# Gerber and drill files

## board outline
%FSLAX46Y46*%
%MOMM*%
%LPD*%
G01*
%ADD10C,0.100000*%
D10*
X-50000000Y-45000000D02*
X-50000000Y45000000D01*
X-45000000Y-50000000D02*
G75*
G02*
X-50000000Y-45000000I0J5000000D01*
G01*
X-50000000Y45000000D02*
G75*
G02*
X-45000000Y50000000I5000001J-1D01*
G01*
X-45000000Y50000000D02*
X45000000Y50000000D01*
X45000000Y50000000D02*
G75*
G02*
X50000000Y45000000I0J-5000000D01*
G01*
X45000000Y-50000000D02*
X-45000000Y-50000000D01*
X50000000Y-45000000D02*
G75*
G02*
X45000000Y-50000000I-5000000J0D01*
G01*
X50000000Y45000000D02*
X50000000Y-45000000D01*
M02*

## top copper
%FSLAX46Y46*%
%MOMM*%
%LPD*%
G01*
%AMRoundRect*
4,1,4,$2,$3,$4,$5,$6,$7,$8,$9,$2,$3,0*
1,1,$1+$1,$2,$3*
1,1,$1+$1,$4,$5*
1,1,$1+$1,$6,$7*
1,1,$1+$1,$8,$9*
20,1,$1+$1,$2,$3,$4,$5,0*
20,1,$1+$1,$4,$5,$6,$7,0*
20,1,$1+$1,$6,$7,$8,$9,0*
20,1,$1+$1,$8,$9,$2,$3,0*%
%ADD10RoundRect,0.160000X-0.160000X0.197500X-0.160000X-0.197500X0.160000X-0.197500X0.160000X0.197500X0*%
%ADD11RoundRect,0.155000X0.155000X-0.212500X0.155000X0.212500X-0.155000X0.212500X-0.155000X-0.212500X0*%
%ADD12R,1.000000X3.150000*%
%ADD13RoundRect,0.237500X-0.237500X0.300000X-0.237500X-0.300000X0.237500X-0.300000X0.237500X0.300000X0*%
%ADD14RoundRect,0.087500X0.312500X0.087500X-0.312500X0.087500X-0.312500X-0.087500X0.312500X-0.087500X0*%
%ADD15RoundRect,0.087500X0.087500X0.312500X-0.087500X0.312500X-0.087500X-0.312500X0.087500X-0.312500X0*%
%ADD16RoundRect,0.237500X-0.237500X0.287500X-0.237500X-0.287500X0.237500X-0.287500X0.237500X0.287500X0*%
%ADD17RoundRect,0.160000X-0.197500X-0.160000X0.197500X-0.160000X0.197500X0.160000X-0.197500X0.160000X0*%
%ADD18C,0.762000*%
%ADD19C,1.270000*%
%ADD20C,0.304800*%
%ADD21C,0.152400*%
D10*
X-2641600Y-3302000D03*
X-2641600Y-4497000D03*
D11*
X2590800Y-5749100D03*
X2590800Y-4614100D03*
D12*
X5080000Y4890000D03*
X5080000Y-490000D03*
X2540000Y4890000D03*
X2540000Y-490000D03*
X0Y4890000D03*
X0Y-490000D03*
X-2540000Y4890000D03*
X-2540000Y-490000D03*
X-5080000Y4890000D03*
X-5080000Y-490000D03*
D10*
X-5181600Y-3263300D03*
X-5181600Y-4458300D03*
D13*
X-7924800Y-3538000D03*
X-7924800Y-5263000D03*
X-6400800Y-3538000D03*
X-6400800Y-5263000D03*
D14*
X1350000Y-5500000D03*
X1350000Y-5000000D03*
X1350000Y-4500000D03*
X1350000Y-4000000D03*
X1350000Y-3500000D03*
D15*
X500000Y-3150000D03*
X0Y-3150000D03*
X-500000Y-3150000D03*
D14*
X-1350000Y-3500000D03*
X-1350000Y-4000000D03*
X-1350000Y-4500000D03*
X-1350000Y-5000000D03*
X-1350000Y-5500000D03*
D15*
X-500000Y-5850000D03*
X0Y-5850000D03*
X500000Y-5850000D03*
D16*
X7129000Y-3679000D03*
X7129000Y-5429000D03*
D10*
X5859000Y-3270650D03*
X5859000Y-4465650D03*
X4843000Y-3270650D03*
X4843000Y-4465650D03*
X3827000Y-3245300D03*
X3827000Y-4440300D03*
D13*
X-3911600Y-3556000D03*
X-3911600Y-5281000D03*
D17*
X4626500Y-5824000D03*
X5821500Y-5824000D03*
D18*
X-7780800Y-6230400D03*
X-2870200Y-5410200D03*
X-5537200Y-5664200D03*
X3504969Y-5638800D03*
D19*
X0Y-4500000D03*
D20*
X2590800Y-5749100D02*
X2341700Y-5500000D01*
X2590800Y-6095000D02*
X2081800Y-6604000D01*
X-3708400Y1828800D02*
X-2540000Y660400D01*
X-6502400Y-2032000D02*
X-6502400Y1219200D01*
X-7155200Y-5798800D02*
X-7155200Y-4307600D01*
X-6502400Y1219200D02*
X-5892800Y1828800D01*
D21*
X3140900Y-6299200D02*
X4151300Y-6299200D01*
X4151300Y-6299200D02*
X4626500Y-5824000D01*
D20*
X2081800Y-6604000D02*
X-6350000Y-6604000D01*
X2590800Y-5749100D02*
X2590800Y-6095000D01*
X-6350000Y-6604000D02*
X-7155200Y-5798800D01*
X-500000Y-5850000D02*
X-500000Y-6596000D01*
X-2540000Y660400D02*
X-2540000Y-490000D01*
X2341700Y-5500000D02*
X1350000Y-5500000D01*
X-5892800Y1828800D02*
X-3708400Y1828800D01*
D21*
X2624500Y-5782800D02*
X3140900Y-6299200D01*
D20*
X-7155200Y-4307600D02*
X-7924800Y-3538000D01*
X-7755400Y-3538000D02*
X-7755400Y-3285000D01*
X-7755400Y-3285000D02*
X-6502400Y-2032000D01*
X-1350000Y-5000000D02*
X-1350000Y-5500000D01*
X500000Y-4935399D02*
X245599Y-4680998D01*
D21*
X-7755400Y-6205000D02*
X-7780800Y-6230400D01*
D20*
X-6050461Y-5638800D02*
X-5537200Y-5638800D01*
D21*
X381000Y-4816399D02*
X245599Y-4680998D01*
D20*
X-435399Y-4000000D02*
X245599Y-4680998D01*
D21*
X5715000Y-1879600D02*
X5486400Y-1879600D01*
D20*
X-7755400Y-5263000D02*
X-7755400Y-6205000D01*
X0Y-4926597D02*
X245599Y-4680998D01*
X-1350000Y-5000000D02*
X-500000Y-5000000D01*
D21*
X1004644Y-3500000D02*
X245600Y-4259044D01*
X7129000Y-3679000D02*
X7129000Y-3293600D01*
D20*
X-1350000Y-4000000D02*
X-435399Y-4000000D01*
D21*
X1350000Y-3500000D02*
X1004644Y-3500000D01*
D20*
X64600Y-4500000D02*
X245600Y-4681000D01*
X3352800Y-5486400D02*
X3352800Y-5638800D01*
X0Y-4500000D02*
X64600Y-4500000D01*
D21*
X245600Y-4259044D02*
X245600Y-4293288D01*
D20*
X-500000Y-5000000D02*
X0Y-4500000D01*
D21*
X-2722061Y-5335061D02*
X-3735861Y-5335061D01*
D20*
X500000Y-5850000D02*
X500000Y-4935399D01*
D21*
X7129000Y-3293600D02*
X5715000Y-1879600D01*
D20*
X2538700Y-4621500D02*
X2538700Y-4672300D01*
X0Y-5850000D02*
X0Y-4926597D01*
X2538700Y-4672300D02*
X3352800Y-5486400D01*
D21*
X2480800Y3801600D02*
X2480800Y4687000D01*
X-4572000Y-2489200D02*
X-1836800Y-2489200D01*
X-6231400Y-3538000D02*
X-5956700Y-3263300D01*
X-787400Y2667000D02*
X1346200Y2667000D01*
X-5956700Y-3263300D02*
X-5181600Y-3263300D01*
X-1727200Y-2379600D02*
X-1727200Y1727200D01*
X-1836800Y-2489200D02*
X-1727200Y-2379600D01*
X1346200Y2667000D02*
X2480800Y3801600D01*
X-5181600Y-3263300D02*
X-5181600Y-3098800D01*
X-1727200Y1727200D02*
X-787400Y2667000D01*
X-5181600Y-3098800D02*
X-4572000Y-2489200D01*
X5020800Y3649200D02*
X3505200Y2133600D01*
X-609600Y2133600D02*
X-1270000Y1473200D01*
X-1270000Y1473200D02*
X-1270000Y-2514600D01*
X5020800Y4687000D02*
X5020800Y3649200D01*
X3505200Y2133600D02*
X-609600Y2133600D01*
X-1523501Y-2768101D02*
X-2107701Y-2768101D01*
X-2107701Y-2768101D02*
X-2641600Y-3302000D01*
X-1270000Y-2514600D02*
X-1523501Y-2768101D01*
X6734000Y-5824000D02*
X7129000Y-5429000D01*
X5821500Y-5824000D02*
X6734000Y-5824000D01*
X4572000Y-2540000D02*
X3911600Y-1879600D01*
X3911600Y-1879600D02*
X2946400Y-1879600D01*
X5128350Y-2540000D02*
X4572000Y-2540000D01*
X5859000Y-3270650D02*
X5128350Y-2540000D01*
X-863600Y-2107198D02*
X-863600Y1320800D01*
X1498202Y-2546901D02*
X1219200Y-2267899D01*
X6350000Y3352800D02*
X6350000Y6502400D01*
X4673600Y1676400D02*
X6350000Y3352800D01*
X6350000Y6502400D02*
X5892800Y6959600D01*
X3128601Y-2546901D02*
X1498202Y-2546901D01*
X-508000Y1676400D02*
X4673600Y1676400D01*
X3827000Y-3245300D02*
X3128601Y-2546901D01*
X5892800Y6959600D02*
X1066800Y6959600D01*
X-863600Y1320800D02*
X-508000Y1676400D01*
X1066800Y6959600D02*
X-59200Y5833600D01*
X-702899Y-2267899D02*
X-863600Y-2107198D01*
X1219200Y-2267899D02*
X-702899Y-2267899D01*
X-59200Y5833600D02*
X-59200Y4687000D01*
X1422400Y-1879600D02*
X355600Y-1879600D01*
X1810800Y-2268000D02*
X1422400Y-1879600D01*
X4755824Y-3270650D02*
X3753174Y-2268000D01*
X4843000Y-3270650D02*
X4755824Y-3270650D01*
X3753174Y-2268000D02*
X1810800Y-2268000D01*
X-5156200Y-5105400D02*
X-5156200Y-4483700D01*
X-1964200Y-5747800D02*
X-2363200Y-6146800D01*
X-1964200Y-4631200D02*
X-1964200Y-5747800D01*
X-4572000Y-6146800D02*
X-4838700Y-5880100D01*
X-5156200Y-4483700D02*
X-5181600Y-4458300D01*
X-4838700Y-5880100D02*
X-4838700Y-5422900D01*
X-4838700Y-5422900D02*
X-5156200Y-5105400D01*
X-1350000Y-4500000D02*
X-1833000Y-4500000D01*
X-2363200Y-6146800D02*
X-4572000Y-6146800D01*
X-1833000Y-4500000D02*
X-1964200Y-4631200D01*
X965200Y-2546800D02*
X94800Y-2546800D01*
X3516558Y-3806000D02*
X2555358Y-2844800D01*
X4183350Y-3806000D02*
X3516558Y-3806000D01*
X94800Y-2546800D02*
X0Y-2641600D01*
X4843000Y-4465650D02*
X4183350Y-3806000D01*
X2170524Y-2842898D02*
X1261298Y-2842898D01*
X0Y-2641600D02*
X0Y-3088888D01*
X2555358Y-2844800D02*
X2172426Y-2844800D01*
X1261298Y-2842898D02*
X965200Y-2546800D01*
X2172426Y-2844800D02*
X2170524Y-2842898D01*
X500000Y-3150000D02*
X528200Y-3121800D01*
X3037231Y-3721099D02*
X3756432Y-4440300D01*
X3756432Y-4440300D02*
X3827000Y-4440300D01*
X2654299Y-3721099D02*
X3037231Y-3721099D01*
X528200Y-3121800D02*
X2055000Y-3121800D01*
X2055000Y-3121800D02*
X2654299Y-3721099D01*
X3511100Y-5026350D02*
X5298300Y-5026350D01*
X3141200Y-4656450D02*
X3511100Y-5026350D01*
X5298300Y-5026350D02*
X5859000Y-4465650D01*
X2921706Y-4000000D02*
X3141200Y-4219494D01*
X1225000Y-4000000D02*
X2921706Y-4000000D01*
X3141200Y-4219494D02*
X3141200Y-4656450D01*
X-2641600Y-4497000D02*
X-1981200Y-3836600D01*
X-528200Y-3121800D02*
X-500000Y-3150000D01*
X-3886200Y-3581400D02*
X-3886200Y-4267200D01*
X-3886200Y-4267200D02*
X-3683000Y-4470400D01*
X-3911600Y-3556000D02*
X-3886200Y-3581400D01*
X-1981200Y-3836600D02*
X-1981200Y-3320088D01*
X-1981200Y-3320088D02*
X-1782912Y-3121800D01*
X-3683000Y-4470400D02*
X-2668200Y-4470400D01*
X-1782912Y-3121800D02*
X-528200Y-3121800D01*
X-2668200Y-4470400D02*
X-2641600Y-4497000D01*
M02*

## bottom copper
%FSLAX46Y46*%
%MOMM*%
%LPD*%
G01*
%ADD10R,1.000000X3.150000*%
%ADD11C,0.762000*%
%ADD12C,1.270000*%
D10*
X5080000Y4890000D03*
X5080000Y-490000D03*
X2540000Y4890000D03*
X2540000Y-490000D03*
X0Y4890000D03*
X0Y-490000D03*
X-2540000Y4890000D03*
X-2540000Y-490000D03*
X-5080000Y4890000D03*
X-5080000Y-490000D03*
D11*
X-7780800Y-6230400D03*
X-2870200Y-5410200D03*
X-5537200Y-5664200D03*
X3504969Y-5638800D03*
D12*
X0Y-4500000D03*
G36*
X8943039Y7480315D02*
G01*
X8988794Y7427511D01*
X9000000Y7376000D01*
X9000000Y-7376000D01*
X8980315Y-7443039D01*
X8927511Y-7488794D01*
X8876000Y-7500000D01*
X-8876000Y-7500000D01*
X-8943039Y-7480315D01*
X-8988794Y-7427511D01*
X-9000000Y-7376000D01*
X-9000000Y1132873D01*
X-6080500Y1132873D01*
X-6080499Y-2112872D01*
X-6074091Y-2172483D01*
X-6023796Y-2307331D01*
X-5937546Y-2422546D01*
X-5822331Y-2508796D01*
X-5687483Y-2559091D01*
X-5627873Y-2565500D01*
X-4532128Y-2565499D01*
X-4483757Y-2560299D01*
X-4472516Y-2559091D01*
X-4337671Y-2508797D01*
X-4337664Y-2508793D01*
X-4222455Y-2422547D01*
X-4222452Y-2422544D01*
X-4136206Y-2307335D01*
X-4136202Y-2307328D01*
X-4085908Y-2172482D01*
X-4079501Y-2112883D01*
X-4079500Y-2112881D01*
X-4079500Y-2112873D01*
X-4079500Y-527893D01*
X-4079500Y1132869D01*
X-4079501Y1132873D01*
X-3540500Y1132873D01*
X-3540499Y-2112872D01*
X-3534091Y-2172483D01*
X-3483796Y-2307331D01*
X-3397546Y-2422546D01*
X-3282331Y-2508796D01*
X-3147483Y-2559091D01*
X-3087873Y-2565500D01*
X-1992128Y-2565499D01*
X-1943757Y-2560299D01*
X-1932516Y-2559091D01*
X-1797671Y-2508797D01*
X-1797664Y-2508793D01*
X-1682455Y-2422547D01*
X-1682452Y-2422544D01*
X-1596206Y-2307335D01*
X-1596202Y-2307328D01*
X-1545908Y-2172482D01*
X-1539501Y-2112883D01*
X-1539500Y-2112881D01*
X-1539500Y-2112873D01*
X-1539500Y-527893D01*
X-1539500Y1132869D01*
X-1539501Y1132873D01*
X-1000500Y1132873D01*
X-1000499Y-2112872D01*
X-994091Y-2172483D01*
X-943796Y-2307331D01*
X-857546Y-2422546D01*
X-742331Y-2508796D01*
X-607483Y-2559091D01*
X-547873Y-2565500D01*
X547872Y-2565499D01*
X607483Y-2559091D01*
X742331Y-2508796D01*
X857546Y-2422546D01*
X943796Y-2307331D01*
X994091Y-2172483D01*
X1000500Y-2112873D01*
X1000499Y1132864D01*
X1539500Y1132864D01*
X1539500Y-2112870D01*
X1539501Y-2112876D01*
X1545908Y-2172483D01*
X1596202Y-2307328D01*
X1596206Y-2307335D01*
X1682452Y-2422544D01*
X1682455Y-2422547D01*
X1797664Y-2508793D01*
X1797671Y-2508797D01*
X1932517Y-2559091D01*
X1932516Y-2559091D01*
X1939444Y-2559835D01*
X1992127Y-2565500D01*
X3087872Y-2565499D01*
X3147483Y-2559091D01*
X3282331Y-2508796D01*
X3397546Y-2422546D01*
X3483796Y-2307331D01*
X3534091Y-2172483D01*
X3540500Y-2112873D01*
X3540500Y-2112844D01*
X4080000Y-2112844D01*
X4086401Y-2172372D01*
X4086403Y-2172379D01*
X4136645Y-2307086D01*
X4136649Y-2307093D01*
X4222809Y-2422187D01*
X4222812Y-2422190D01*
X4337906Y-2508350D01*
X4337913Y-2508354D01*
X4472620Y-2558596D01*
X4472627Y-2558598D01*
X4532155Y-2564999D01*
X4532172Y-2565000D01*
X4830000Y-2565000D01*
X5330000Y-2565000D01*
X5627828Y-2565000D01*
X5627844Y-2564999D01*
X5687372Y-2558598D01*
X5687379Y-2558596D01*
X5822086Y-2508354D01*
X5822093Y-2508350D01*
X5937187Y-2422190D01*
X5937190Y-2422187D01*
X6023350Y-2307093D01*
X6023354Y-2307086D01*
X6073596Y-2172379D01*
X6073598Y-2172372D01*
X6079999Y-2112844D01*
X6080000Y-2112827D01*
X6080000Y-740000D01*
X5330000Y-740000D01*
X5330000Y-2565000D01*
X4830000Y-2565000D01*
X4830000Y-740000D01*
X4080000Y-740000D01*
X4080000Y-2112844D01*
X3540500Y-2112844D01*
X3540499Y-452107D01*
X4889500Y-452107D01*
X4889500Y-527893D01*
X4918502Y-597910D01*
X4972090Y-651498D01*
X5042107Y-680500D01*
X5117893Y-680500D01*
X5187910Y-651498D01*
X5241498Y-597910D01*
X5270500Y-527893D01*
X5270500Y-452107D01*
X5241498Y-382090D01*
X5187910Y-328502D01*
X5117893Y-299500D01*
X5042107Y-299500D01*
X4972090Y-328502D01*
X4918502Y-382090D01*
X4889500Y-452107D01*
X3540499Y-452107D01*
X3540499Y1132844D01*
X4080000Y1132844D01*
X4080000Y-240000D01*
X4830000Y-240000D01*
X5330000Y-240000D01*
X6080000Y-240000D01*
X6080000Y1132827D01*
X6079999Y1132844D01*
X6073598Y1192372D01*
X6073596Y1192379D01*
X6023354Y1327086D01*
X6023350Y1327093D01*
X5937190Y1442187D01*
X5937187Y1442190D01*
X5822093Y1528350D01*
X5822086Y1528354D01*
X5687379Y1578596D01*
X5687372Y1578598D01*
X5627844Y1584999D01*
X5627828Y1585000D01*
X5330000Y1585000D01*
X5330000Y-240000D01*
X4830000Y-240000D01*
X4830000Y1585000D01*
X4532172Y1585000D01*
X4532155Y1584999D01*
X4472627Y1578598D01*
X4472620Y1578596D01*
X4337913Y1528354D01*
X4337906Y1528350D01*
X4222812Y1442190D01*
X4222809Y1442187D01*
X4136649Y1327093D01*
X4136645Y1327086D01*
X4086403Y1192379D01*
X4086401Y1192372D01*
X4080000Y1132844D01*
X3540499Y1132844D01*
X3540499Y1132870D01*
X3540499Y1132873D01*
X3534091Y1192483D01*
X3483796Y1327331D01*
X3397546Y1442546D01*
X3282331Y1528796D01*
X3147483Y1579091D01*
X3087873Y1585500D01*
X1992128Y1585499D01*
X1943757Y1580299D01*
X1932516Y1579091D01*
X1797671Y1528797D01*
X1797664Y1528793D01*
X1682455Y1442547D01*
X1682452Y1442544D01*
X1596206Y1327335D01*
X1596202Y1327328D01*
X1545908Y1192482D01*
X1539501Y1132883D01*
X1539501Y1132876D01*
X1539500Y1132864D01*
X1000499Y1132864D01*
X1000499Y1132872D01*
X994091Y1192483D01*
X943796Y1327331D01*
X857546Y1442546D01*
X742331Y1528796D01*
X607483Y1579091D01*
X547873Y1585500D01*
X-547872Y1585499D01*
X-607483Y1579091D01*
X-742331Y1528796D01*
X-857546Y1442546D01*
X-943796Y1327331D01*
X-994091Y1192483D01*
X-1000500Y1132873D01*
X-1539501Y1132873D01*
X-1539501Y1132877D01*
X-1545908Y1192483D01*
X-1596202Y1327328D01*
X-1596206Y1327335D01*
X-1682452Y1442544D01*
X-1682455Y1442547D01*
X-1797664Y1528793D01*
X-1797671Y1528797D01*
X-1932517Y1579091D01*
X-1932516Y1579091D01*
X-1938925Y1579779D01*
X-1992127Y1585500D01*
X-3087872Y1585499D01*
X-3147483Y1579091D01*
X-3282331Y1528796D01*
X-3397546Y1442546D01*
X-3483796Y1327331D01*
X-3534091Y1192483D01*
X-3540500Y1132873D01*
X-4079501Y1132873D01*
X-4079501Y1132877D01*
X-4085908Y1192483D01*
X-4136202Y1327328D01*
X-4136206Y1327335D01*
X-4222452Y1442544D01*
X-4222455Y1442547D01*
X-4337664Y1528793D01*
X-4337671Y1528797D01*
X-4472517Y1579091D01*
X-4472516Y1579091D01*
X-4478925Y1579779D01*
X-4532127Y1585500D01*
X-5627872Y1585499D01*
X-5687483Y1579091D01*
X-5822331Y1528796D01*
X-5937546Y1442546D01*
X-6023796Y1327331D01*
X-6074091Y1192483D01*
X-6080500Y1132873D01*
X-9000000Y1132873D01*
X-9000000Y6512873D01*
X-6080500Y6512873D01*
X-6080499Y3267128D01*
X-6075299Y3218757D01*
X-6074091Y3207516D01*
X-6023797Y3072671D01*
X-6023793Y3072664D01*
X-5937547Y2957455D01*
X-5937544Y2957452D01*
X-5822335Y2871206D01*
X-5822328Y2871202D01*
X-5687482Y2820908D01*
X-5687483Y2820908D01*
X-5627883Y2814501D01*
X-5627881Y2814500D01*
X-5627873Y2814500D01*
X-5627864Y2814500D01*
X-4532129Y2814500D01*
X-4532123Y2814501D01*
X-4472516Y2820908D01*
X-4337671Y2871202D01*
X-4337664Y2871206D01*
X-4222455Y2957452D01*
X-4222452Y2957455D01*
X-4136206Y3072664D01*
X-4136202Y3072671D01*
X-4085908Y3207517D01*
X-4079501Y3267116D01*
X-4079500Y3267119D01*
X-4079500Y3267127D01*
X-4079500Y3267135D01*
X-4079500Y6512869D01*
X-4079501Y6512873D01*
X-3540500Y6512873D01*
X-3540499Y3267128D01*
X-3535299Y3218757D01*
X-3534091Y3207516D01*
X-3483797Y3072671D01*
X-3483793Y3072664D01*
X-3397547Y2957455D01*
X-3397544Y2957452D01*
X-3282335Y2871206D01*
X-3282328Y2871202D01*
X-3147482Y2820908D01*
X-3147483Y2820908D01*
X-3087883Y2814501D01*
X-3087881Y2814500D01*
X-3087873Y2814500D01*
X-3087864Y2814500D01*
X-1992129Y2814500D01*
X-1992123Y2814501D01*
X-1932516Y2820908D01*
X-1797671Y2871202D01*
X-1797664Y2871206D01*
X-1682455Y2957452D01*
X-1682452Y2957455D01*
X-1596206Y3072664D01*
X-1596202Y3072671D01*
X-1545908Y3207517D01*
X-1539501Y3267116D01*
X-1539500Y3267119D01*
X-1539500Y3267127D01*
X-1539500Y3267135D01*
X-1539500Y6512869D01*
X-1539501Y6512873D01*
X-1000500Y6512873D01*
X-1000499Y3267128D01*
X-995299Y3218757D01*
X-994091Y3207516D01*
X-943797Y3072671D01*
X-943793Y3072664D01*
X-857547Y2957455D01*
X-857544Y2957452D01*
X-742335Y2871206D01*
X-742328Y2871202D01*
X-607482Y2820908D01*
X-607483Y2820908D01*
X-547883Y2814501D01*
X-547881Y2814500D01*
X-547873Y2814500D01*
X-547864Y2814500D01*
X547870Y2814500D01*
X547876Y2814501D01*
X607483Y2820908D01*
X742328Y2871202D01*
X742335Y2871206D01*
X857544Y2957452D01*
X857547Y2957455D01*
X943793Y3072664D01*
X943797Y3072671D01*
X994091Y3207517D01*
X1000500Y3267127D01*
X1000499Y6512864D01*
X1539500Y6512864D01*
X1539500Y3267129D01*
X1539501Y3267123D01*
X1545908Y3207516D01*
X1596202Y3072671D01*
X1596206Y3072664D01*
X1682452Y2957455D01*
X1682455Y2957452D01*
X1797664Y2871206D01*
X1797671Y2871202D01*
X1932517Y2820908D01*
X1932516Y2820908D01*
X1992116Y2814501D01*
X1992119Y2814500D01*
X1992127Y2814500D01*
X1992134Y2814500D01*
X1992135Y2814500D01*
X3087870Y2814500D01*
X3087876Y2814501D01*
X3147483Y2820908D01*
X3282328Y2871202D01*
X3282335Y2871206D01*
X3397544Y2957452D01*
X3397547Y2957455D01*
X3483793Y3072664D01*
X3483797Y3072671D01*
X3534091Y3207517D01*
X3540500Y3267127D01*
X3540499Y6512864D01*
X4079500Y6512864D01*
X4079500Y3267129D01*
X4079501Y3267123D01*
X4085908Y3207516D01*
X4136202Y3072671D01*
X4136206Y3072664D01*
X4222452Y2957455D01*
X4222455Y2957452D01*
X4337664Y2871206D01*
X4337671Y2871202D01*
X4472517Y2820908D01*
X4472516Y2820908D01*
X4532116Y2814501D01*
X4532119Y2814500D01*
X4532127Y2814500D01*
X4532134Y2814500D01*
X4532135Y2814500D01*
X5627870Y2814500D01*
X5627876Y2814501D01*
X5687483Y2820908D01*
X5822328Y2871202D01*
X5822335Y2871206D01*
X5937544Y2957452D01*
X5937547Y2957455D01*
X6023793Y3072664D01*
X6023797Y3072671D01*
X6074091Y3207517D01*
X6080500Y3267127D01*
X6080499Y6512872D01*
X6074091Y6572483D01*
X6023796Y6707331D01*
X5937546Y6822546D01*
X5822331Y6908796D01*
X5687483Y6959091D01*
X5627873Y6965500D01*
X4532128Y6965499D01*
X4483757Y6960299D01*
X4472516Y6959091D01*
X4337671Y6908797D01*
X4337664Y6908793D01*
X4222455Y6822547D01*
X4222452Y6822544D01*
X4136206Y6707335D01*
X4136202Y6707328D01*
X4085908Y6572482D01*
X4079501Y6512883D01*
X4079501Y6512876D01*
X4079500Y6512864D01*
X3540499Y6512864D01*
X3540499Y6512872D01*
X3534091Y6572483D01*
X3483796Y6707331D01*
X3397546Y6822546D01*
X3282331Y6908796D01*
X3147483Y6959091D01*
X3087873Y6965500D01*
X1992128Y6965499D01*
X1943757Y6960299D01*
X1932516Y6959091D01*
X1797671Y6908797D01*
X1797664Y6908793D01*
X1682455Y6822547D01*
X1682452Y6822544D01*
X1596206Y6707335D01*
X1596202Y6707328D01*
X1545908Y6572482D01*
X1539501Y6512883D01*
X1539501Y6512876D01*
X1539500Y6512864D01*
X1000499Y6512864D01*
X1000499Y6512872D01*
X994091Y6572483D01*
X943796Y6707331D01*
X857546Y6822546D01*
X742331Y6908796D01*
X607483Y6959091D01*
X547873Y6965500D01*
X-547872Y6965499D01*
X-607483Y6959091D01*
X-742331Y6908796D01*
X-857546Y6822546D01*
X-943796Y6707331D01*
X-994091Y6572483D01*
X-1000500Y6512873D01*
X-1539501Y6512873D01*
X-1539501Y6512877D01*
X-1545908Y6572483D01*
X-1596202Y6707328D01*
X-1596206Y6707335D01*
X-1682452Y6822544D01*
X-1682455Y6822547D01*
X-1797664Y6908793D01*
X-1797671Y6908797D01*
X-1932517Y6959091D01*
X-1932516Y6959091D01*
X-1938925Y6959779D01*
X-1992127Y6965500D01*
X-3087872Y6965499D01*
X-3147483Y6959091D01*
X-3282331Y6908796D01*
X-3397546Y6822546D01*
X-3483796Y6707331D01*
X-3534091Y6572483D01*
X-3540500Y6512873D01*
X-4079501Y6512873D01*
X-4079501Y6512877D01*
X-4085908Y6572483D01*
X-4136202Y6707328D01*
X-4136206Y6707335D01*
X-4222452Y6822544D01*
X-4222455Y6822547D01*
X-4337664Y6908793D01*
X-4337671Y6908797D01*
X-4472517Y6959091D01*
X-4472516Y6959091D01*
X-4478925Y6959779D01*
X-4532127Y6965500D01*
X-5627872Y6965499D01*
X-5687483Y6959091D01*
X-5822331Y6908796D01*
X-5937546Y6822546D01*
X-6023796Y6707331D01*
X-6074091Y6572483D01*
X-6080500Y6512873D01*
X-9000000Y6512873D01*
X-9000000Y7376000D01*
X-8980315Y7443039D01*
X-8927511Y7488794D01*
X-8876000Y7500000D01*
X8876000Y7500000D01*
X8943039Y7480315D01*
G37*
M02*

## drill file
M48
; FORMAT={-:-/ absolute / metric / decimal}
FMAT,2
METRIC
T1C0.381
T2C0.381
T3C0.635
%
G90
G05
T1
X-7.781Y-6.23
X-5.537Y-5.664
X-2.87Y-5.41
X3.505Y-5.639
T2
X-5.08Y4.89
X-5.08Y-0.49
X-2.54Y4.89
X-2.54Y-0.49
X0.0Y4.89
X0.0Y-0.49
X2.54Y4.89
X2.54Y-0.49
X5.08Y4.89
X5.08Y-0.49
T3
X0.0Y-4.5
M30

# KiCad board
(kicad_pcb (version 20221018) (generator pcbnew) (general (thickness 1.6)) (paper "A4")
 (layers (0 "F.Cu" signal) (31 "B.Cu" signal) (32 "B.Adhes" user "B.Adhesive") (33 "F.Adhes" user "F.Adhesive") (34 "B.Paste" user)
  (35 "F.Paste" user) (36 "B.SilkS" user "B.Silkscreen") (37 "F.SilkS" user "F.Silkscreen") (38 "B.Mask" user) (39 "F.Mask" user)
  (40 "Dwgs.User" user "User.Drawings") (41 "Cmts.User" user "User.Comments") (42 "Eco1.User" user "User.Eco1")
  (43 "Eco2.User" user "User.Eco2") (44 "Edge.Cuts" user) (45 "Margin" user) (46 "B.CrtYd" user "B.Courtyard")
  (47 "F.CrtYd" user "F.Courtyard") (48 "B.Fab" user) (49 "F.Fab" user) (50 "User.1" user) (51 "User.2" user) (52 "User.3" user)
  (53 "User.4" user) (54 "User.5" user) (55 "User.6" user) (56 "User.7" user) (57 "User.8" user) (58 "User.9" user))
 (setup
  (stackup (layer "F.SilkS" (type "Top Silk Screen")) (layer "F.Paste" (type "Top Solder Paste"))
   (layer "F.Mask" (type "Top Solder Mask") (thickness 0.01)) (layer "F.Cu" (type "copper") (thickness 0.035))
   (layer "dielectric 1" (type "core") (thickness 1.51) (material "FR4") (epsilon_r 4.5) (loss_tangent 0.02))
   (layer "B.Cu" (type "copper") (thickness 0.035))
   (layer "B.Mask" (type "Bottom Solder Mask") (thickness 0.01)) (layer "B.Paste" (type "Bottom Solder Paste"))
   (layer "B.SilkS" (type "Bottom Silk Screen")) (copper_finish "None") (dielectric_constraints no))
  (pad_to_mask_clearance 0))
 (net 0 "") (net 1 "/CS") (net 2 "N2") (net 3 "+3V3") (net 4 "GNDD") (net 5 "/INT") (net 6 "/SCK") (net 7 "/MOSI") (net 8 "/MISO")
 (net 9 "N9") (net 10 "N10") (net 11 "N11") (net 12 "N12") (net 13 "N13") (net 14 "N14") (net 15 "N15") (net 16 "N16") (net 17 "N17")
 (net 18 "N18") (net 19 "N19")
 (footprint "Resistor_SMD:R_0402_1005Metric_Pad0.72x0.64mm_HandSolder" (layer "F.Cu") (at -2.6416 3.8995 -90)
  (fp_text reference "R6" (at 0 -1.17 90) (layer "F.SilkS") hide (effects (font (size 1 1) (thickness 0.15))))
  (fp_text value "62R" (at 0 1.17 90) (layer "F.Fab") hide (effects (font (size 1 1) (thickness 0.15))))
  (pad "1" smd roundrect (at -0.5975 0 270) (size 0.715 0.64) (layers "F.Cu" "F.Paste" "F.Mask") (roundrect_rratio 0.25) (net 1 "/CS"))
  (pad "2" smd roundrect (at 0.5975 0 270) (size 0.715 0.64) (layers "F.Cu" "F.Paste" "F.Mask") (roundrect_rratio 0.25) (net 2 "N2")))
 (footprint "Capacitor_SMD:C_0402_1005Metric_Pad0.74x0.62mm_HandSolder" (layer "F.Cu") (at 2.5908 5.1816 90)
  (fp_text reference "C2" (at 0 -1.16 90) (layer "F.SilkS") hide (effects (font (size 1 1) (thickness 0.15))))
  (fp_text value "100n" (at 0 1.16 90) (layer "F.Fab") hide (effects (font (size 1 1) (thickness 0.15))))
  (pad "1" smd roundrect (at -0.5675 0 90) (size 0.735 0.62) (layers "F.Cu" "F.Paste" "F.Mask") (roundrect_rratio 0.25) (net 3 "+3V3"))
  (pad "2" smd roundrect (at 0.5675 0 90) (size 0.735 0.62) (layers "F.Cu" "F.Paste" "F.Mask") (roundrect_rratio 0.25) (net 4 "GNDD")))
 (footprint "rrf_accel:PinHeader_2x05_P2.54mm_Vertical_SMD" (layer "F.Cu") (at 0 -2.2 -90)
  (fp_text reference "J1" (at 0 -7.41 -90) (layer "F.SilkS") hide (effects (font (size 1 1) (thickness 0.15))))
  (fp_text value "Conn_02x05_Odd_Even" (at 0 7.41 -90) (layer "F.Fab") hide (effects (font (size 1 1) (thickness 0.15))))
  (pad "1" thru_hole rect (at -2.69 -5.08 270) (size 3.15 1) (drill 0.381) (layers "*.Cu" "F.Paste" "F.Mask") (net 1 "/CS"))
  (pad "2" thru_hole rect (at 2.69 -5.08 270) (size 3.15 1) (drill 0.381) (layers "*.Cu" "F.Paste" "F.Mask") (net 4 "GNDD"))
  (pad "3" thru_hole rect (at -2.69 -2.54 270) (size 3.15 1) (drill 0.381) (layers "*.Cu" "F.Paste" "F.Mask") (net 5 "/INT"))
  (pad "4" thru_hole rect (at 2.69 -2.54 270) (size 3.15 1) (drill 0.381) (layers "*.Cu" "F.Paste" "F.Mask") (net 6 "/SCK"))
  (pad "5" thru_hole rect (at -2.69 0 270) (size 3.15 1) (drill 0.381) (layers "*.Cu" "F.Paste" "F.Mask") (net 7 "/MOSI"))
  (pad "6" thru_hole rect (at 2.69 0 270) (size 3.15 1) (drill 0.381) (layers "*.Cu" "F.Paste" "F.Mask") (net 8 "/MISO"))
  (pad "7" thru_hole rect (at -2.69 2.54 270) (size 3.15 1) (drill 0.381) (layers "*.Cu" "F.Paste" "F.Mask") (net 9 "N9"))
  (pad "8" thru_hole rect (at 2.69 2.54 270) (size 3.15 1) (drill 0.381) (layers "*.Cu" "F.Paste" "F.Mask") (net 3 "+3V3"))
  (pad "9" thru_hole rect (at -2.69 5.08 270) (size 3.15 1) (drill 0.381) (layers "*.Cu" "F.Paste" "F.Mask") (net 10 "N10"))
  (pad "10" thru_hole rect (at 2.69 5.08 270) (size 3.15 1) (drill 0.381) (layers "*.Cu" "F.Paste" "F.Mask") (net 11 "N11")))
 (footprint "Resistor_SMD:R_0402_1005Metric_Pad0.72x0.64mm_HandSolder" (layer "F.Cu") (at -5.1816 3.8608 -90)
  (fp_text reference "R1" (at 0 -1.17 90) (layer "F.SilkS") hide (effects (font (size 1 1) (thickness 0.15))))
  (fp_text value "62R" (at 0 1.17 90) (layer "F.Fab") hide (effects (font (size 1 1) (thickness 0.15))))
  (pad "1" smd roundrect (at -0.5975 0 270) (size 0.715 0.64) (layers "F.Cu" "F.Paste" "F.Mask") (roundrect_rratio 0.25) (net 5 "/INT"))
  (pad "2" smd roundrect (at 0.5975 0 270) (size 0.715 0.64) (layers "F.Cu" "F.Paste" "F.Mask") (roundrect_rratio 0.25) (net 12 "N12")))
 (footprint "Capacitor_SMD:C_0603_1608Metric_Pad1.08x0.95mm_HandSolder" (layer "F.Cu") (at -7.9248 4.4005 -90)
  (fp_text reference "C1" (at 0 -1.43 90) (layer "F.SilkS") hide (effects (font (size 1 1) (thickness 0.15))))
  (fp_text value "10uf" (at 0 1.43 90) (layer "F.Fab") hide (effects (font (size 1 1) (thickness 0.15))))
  (pad "1" smd roundrect (at -0.8625 0 270) (size 1.075 0.95) (layers "F.Cu" "F.Paste" "F.Mask") (roundrect_rratio 0.25) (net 3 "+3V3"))
  (pad "2" smd roundrect (at 0.8625 0 270) (size 1.075 0.95) (layers "F.Cu" "F.Paste" "F.Mask") (roundrect_rratio 0.25) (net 4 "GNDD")))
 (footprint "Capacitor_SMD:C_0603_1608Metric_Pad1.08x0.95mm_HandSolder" (layer "F.Cu") (at -6.4008 4.4005 -90)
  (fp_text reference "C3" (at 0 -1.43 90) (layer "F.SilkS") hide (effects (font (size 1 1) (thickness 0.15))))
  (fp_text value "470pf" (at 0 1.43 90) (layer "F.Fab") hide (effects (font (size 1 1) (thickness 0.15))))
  (pad "1" smd roundrect (at -0.8625 0 270) (size 1.075 0.95) (layers "F.Cu" "F.Paste" "F.Mask") (roundrect_rratio 0.25) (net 5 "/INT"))
  (pad "2" smd roundrect (at 0.8625 0 270) (size 1.075 0.95) (layers "F.Cu" "F.Paste" "F.Mask") (roundrect_rratio 0.25) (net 4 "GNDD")))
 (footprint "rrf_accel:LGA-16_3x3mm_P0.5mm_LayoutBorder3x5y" (layer "F.Cu") (at 0 4.5 180)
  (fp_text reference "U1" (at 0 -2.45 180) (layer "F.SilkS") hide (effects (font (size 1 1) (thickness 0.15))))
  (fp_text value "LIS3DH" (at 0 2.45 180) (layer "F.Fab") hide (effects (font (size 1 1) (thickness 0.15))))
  (pad "1" smd roundrect (at -1.35 -1 180) (size 0.8 0.35) (layers "F.Cu" "F.Paste" "F.Mask") (roundrect_rratio 0.25) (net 3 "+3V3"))
  (pad "2" smd roundrect (at -1.35 -0.5 180) (size 0.8 0.35) (layers "F.Cu" "F.Paste" "F.Mask") (roundrect_rratio 0.25) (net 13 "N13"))
  (pad "3" smd roundrect (at -1.35 0 180) (size 0.8 0.35) (layers "F.Cu" "F.Paste" "F.Mask") (roundrect_rratio 0.25) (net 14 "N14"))
  (pad "4" smd roundrect (at -1.35 0.5 180) (size 0.8 0.35) (layers "F.Cu" "F.Paste" "F.Mask") (roundrect_rratio 0.25) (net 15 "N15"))
  (pad "5" smd roundrect (at -1.35 1 180) (size 0.8 0.35) (layers "F.Cu" "F.Paste" "F.Mask") (roundrect_rratio 0.25) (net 4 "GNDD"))
  (pad "6" smd roundrect (at -0.5 1.35 180) (size 0.35 0.8) (layers "F.Cu" "F.Paste" "F.Mask") (roundrect_rratio 0.25) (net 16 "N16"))
  (pad "7" smd roundrect (at 0 1.35 180) (size 0.35 0.8) (layers "F.Cu" "F.Paste" "F.Mask") (roundrect_rratio 0.25) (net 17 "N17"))
  (pad "8" smd roundrect (at 0.5 1.35 180) (size 0.35 0.8) (layers "F.Cu" "F.Paste" "F.Mask") (roundrect_rratio 0.25) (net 2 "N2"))
  (pad "9" smd roundrect (at 1.35 1 180) (size 0.8 0.35) (layers "F.Cu" "F.Paste" "F.Mask") (roundrect_rratio 0.25) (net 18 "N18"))
  (pad "10" smd roundrect (at 1.35 0.5 180) (size 0.8 0.35) (layers "F.Cu" "F.Paste" "F.Mask") (roundrect_rratio 0.25) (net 4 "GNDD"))
  (pad "11" smd roundrect (at 1.35 0 180) (size 0.8 0.35) (layers "F.Cu" "F.Paste" "F.Mask") (roundrect_rratio 0.25) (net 12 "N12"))
  (pad "12" smd roundrect (at 1.35 -0.5 180) (size 0.8 0.35) (layers "F.Cu" "F.Paste" "F.Mask") (roundrect_rratio 0.25) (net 4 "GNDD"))
  (pad "13" smd roundrect (at 1.35 -1 180) (size 0.8 0.35) (layers "F.Cu" "F.Paste" "F.Mask") (roundrect_rratio 0.25) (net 4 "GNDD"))
  (pad "14" smd roundrect (at 0.5 -1.35 180) (size 0.35 0.8) (layers "F.Cu" "F.Paste" "F.Mask") (roundrect_rratio 0.25) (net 3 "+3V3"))
  (pad "15" smd roundrect (at 0 -1.35 180) (size 0.35 0.8) (layers "F.Cu" "F.Paste" "F.Mask") (roundrect_rratio 0.25) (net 4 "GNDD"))
  (pad "16" smd roundrect (at -0.5 -1.35 180) (size 0.35 0.8) (layers "F.Cu" "F.Paste" "F.Mask") (roundrect_rratio 0.25) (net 4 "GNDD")))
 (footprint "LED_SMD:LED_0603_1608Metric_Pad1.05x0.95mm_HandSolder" (layer "F.Cu") (at 7.129 4.554 -90)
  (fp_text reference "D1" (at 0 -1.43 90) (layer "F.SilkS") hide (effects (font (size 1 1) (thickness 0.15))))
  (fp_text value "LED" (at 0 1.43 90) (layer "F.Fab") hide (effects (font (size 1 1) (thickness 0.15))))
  (pad "1" smd roundrect (at -0.875 0 270) (size 1.05 0.95) (layers "F.Cu" "F.Paste" "F.Mask") (roundrect_rratio 0.25) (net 4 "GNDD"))
  (pad "2" smd roundrect (at 0.875 0 270) (size 1.05 0.95) (layers "F.Cu" "F.Paste" "F.Mask") (roundrect_rratio 0.25) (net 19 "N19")))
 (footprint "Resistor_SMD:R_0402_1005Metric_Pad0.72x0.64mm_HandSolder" (layer "F.Cu") (at 5.859 3.86815 -90)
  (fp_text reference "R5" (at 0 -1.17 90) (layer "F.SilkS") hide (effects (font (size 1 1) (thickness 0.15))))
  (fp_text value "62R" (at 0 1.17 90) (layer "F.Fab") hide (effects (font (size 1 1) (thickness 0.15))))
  (pad "1" smd roundrect (at -0.5975 0 270) (size 0.715 0.64) (layers "F.Cu" "F.Paste" "F.Mask") (roundrect_rratio 0.25) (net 6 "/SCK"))
  (pad "2" smd roundrect (at 0.5975 0 270) (size 0.715 0.64) (layers "F.Cu" "F.Paste" "F.Mask") (roundrect_rratio 0.25) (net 15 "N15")))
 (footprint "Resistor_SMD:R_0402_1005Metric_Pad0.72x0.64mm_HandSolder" (layer "F.Cu") (at 4.843 3.86815 -90)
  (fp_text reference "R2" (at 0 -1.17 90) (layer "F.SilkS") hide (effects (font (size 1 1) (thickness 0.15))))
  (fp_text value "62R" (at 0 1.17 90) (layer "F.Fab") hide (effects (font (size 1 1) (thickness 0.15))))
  (pad "1" smd roundrect (at -0.5975 0 270) (size 0.715 0.64) (layers "F.Cu" "F.Paste" "F.Mask") (roundrect_rratio 0.25) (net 8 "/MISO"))
  (pad "2" smd roundrect (at 0.5975 0 270) (size 0.715 0.64) (layers "F.Cu" "F.Paste" "F.Mask") (roundrect_rratio 0.25) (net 17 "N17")))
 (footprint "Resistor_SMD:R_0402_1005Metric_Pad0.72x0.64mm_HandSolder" (layer "F.Cu") (at 3.827 3.8428 -90)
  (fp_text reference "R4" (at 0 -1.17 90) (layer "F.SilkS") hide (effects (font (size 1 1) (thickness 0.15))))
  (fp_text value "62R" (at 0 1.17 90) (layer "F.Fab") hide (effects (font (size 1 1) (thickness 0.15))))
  (pad "1" smd roundrect (at -0.5975 0 270) (size 0.715 0.64) (layers "F.Cu" "F.Paste" "F.Mask") (roundrect_rratio 0.25) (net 7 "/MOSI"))
  (pad "2" smd roundrect (at 0.5975 0 270) (size 0.715 0.64) (layers "F.Cu" "F.Paste" "F.Mask") (roundrect_rratio 0.25) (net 16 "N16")))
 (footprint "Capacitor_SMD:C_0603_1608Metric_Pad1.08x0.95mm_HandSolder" (layer "F.Cu") (at -3.9116 4.4185 -90)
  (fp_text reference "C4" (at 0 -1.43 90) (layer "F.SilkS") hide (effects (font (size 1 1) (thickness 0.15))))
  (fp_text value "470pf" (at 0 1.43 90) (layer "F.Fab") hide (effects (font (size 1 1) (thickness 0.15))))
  (pad "1" smd roundrect (at -0.8625 0 270) (size 1.075 0.95) (layers "F.Cu" "F.Paste" "F.Mask") (roundrect_rratio 0.25) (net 2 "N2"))
  (pad "2" smd roundrect (at 0.8625 0 270) (size 1.075 0.95) (layers "F.Cu" "F.Paste" "F.Mask") (roundrect_rratio 0.25) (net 4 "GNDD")))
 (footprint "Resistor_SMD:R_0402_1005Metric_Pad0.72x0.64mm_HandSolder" (layer "F.Cu") (at 5.224 5.824)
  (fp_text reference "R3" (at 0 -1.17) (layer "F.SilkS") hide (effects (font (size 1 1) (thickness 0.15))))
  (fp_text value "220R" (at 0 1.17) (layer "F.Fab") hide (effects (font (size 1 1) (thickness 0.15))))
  (pad "1" smd roundrect (at -0.5975 0) (size 0.715 0.64) (layers "F.Cu" "F.Paste" "F.Mask") (roundrect_rratio 0.25) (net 3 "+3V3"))
  (pad "2" smd roundrect (at 0.5975 0) (size 0.715 0.64) (layers "F.Cu" "F.Paste" "F.Mask") (roundrect_rratio 0.25) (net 19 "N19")))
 (gr_line (start -50 45) (end -50 -45) (stroke (width 0.1) (type solid)) (layer "Edge.Cuts"))
 (gr_arc (start -45 50) (mid -48.535534 48.535534) (end -50 45) (stroke (width 0.1) (type solid)) (layer "Edge.Cuts"))
 (gr_arc (start -50 -45) (mid -48.535534 -48.535533) (end -45 -50) (stroke (width 0.1) (type solid)) (layer "Edge.Cuts"))
 (gr_line (start -45 -50) (end 45 -50) (stroke (width 0.1) (type solid)) (layer "Edge.Cuts"))
 (gr_arc (start 45 -50) (mid 48.535534 -48.535534) (end 50 -45) (stroke (width 0.1) (type solid)) (layer "Edge.Cuts"))
 (gr_line (start 45 50) (end -45 50) (stroke (width 0.1) (type solid)) (layer "Edge.Cuts"))
 (gr_arc (start 50 45) (mid 48.535534 48.535534) (end 45 50) (stroke (width 0.1) (type solid)) (layer "Edge.Cuts"))
 (gr_line (start 50 -45) (end 50 45) (stroke (width 0.1) (type solid)) (layer "Edge.Cuts"))
 (segment (start 2.5908 5.7491) (end 2.3417 5.5) (width 0.3048) (layer "F.Cu") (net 3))
 (segment (start 2.5908 6.095) (end 2.0818 6.604) (width 0.3048) (layer "F.Cu") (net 3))
 (segment (start -3.7084 -1.8288) (end -2.54 -0.6604) (width 0.3048) (layer "F.Cu") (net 3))
 (segment (start -6.5024 2.032) (end -6.5024 -1.2192) (width 0.3048) (layer "F.Cu") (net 3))
 (segment (start -7.1552 5.7988) (end -7.1552 4.3076) (width 0.3048) (layer "F.Cu") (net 3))
 (segment (start -6.5024 -1.2192) (end -5.8928 -1.8288) (width 0.3048) (layer "F.Cu") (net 3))
 (segment (start 3.1409 6.2992) (end 4.1513 6.2992) (width 0.1524) (layer "F.Cu") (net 3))
 (segment (start 4.1513 6.2992) (end 4.6265 5.824) (width 0.1524) (layer "F.Cu") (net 3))
 (segment (start 2.0818 6.604) (end -6.35 6.604) (width 0.3048) (layer "F.Cu") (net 3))
 (segment (start 2.5908 5.7491) (end 2.5908 6.095) (width 0.3048) (layer "F.Cu") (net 3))
 (segment (start -6.35 6.604) (end -7.1552 5.7988) (width 0.3048) (layer "F.Cu") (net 3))
 (segment (start -0.5 5.85) (end -0.5 6.596) (width 0.3048) (layer "F.Cu") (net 3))
 (segment (start -2.54 -0.6604) (end -2.54 0.49) (width 0.3048) (layer "F.Cu") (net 3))
 (segment (start 2.3417 5.5) (end 1.35 5.5) (width 0.3048) (layer "F.Cu") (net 3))
 (segment (start -5.8928 -1.8288) (end -3.7084 -1.8288) (width 0.3048) (layer "F.Cu") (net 3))
 (segment (start 2.6245 5.7828) (end 3.1409 6.2992) (width 0.1524) (layer "F.Cu") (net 3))
 (segment (start -7.1552 4.3076) (end -7.9248 3.538) (width 0.3048) (layer "F.Cu") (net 3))
 (segment (start -7.7554 3.538) (end -7.7554 3.285) (width 0.3048) (layer "F.Cu") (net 3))
 (segment (start -7.7554 3.285) (end -6.5024 2.032) (width 0.3048) (layer "F.Cu") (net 3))
 (segment (start -1.35 5) (end -1.35 5.5) (width 0.3048) (layer "F.Cu") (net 4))
 (segment (start 0.5 4.935399) (end 0.245599 4.680998) (width 0.3048) (layer "F.Cu") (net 4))
 (segment (start -7.7554 6.205) (end -7.7808 6.2304) (width 0.1524) (layer "F.Cu") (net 4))
 (segment (start -6.050461 5.6388) (end -5.5372 5.6388) (width 0.3048) (layer "F.Cu") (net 4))
 (segment (start 0.381 4.816399) (end 0.245599 4.680998) (width 0.1524) (layer "F.Cu") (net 4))
 (segment (start -0.435399 4) (end 0.245599 4.680998) (width 0.3048) (layer "F.Cu") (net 4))
 (segment (start 5.715 1.8796) (end 5.4864 1.8796) (width 0.1524) (layer "F.Cu") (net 4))
 (segment (start -7.7554 5.263) (end -7.7554 6.205) (width 0.3048) (layer "F.Cu") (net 4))
 (segment (start 0 4.926597) (end 0.245599 4.680998) (width 0.3048) (layer "F.Cu") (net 4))
 (segment (start -1.35 5) (end -0.5 5) (width 0.3048) (layer "F.Cu") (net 4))
 (segment (start 1.004644 3.5) (end 0.2456 4.259044) (width 0.1524) (layer "F.Cu") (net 4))
 (segment (start 7.129 3.679) (end 7.129 3.2936) (width 0.1524) (layer "F.Cu") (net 4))
 (segment (start -1.35 4) (end -0.435399 4) (width 0.3048) (layer "F.Cu") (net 4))
 (segment (start 1.35 3.5) (end 1.004644 3.5) (width 0.1524) (layer "F.Cu") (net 4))
 (segment (start 0.0646 4.5) (end 0.2456 4.681) (width 0.3048) (layer "F.Cu") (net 4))
 (segment (start 3.3528 5.4864) (end 3.3528 5.6388) (width 0.3048) (layer "F.Cu") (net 4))
 (segment (start 0 4.5) (end 0.0646 4.5) (width 0.3048) (layer "F.Cu") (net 4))
 (segment (start 0.2456 4.259044) (end 0.2456 4.293288) (width 0.1524) (layer "F.Cu") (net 4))
 (segment (start -0.5 5) (end 0 4.5) (width 0.3048) (layer "F.Cu") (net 4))
 (segment (start -2.722061 5.335061) (end -3.735861 5.335061) (width 0.1524) (layer "F.Cu") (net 4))
 (segment (start 0.5 5.85) (end 0.5 4.935399) (width 0.3048) (layer "F.Cu") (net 4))
 (segment (start 7.129 3.2936) (end 5.715 1.8796) (width 0.1524) (layer "F.Cu") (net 4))
 (segment (start 2.5387 4.6215) (end 2.5387 4.6723) (width 0.3048) (layer "F.Cu") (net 4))
 (segment (start 0 5.85) (end 0 4.926597) (width 0.3048) (layer "F.Cu") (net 4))
 (segment (start 2.5387 4.6723) (end 3.3528 5.4864) (width 0.3048) (layer "F.Cu") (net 4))
 (via (at -7.7808 6.2304) (size 0.762) (drill 0.381) (layers "F.Cu" "B.Cu") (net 4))
 (via (at -2.8702 5.4102) (size 0.762) (drill 0.381) (layers "F.Cu" "B.Cu") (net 4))
 (via (at -5.5372 5.6642) (size 0.762) (drill 0.381) (layers "F.Cu" "B.Cu") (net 4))
 (via (at 3.504969 5.6388) (size 0.762) (drill 0.381) (layers "F.Cu" "B.Cu") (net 4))
 (via (at 0 4.5) (size 1.27) (drill 0.635) (layers "F.Cu" "B.Cu") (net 4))
 (segment (start 2.4808 -3.8016) (end 2.4808 -4.687) (width 0.1524) (layer "F.Cu") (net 5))
 (segment (start -4.572 2.4892) (end -1.8368 2.4892) (width 0.1524) (layer "F.Cu") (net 5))
 (segment (start -6.2314 3.538) (end -5.9567 3.2633) (width 0.1524) (layer "F.Cu") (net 5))
 (segment (start -0.7874 -2.667) (end 1.3462 -2.667) (width 0.1524) (layer "F.Cu") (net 5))
 (segment (start -5.9567 3.2633) (end -5.1816 3.2633) (width 0.1524) (layer "F.Cu") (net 5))
 (segment (start -1.7272 2.3796) (end -1.7272 -1.7272) (width 0.1524) (layer "F.Cu") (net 5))
 (segment (start -1.8368 2.4892) (end -1.7272 2.3796) (width 0.1524) (layer "F.Cu") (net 5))
 (segment (start 1.3462 -2.667) (end 2.4808 -3.8016) (width 0.1524) (layer "F.Cu") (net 5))
 (segment (start -5.1816 3.2633) (end -5.1816 3.0988) (width 0.1524) (layer "F.Cu") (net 5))
 (segment (start -1.7272 -1.7272) (end -0.7874 -2.667) (width 0.1524) (layer "F.Cu") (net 5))
 (segment (start -5.1816 3.0988) (end -4.572 2.4892) (width 0.1524) (layer "F.Cu") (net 5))
 (segment (start 5.0208 -3.6492) (end 3.5052 -2.1336) (width 0.1524) (layer "F.Cu") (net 1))
 (segment (start -0.6096 -2.1336) (end -1.27 -1.4732) (width 0.1524) (layer "F.Cu") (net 1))
 (segment (start -1.27 -1.4732) (end -1.27 2.5146) (width 0.1524) (layer "F.Cu") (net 1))
 (segment (start 5.0208 -4.687) (end 5.0208 -3.6492) (width 0.1524) (layer "F.Cu") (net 1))
 (segment (start 3.5052 -2.1336) (end -0.6096 -2.1336) (width 0.1524) (layer "F.Cu") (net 1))
 (segment (start -1.523501 2.768101) (end -2.107701 2.768101) (width 0.1524) (layer "F.Cu") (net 1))
 (segment (start -2.107701 2.768101) (end -2.6416 3.302) (width 0.1524) (layer "F.Cu") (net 1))
 (segment (start -1.27 2.5146) (end -1.523501 2.768101) (width 0.1524) (layer "F.Cu") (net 1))
 (segment (start 6.734 5.824) (end 7.129 5.429) (width 0.1524) (layer "F.Cu") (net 19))
 (segment (start 5.8215 5.824) (end 6.734 5.824) (width 0.1524) (layer "F.Cu") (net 19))
 (segment (start 4.572 2.54) (end 3.9116 1.8796) (width 0.1524) (layer "F.Cu") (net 6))
 (segment (start 3.9116 1.8796) (end 2.9464 1.8796) (width 0.1524) (layer "F.Cu") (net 6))
 (segment (start 5.12835 2.54) (end 4.572 2.54) (width 0.1524) (layer "F.Cu") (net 6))
 (segment (start 5.859 3.27065) (end 5.12835 2.54) (width 0.1524) (layer "F.Cu") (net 6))
 (segment (start -0.8636 2.107198) (end -0.8636 -1.3208) (width 0.1524) (layer "F.Cu") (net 7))
 (segment (start 1.498202 2.546901) (end 1.2192 2.267899) (width 0.1524) (layer "F.Cu") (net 7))
 (segment (start 6.35 -3.3528) (end 6.35 -6.5024) (width 0.1524) (layer "F.Cu") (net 7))
 (segment (start 4.6736 -1.6764) (end 6.35 -3.3528) (width 0.1524) (layer "F.Cu") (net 7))
 (segment (start 6.35 -6.5024) (end 5.8928 -6.9596) (width 0.1524) (layer "F.Cu") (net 7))
 (segment (start 3.128601 2.546901) (end 1.498202 2.546901) (width 0.1524) (layer "F.Cu") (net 7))
 (segment (start -0.508 -1.6764) (end 4.6736 -1.6764) (width 0.1524) (layer "F.Cu") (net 7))
 (segment (start 3.827 3.2453) (end 3.128601 2.546901) (width 0.1524) (layer "F.Cu") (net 7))
 (segment (start 5.8928 -6.9596) (end 1.0668 -6.9596) (width 0.1524) (layer "F.Cu") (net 7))
 (segment (start -0.8636 -1.3208) (end -0.508 -1.6764) (width 0.1524) (layer "F.Cu") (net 7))
 (segment (start 1.0668 -6.9596) (end -0.0592 -5.8336) (width 0.1524) (layer "F.Cu") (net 7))
 (segment (start -0.702899 2.267899) (end -0.8636 2.107198) (width 0.1524) (layer "F.Cu") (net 7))
 (segment (start 1.2192 2.267899) (end -0.702899 2.267899) (width 0.1524) (layer "F.Cu") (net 7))
 (segment (start -0.0592 -5.8336) (end -0.0592 -4.687) (width 0.1524) (layer "F.Cu") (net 7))
 (segment (start 1.4224 1.8796) (end 0.3556 1.8796) (width 0.1524) (layer "F.Cu") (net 8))
 (segment (start 1.8108 2.268) (end 1.4224 1.8796) (width 0.1524) (layer "F.Cu") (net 8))
 (segment (start 4.755824 3.27065) (end 3.753174 2.268) (width 0.1524) (layer "F.Cu") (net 8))
 (segment (start 4.843 3.27065) (end 4.755824 3.27065) (width 0.1524) (layer "F.Cu") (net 8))
 (segment (start 3.753174 2.268) (end 1.8108 2.268) (width 0.1524) (layer "F.Cu") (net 8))
 (segment (start -5.1562 5.1054) (end -5.1562 4.4837) (width 0.1524) (layer "F.Cu") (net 12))
 (segment (start -1.9642 5.7478) (end -2.3632 6.1468) (width 0.1524) (layer "F.Cu") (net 12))
 (segment (start -1.9642 4.6312) (end -1.9642 5.7478) (width 0.1524) (layer "F.Cu") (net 12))
 (segment (start -4.572 6.1468) (end -4.8387 5.8801) (width 0.1524) (layer "F.Cu") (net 12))
 (segment (start -5.1562 4.4837) (end -5.1816 4.4583) (width 0.1524) (layer "F.Cu") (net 12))
 (segment (start -4.8387 5.8801) (end -4.8387 5.4229) (width 0.1524) (layer "F.Cu") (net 12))
 (segment (start -4.8387 5.4229) (end -5.1562 5.1054) (width 0.1524) (layer "F.Cu") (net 12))
 (segment (start -1.35 4.5) (end -1.833 4.5) (width 0.1524) (layer "F.Cu") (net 12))
 (segment (start -2.3632 6.1468) (end -4.572 6.1468) (width 0.1524) (layer "F.Cu") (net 12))
 (segment (start -1.833 4.5) (end -1.9642 4.6312) (width 0.1524) (layer "F.Cu") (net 12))
 (segment (start 0.9652 2.5468) (end 0.0948 2.5468) (width 0.1524) (layer "F.Cu") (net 17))
 (segment (start 3.516558 3.806) (end 2.555358 2.8448) (width 0.1524) (layer "F.Cu") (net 17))
 (segment (start 4.18335 3.806) (end 3.516558 3.806) (width 0.1524) (layer "F.Cu") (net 17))
 (segment (start 0.0948 2.5468) (end 0 2.6416) (width 0.1524) (layer "F.Cu") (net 17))
 (segment (start 4.843 4.46565) (end 4.18335 3.806) (width 0.1524) (layer "F.Cu") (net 17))
 (segment (start 2.170524 2.842898) (end 1.261298 2.842898) (width 0.1524) (layer "F.Cu") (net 17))
 (segment (start 0 2.6416) (end 0 3.088888) (width 0.1524) (layer "F.Cu") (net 17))
 (segment (start 2.555358 2.8448) (end 2.172426 2.8448) (width 0.1524) (layer "F.Cu") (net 17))
 (segment (start 1.261298 2.842898) (end 0.9652 2.5468) (width 0.1524) (layer "F.Cu") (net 17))
 (segment (start 2.172426 2.8448) (end 2.170524 2.842898) (width 0.1524) (layer "F.Cu") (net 17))
 (segment (start 0.5 3.15) (end 0.5282 3.1218) (width 0.1524) (layer "F.Cu") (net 16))
 (segment (start 3.037231 3.721099) (end 3.756432 4.4403) (width 0.1524) (layer "F.Cu") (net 16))
 (segment (start 3.756432 4.4403) (end 3.827 4.4403) (width 0.1524) (layer "F.Cu") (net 16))
 (segment (start 2.654299 3.721099) (end 3.037231 3.721099) (width 0.1524) (layer "F.Cu") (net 16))
 (segment (start 0.5282 3.1218) (end 2.055 3.1218) (width 0.1524) (layer "F.Cu") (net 16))
 (segment (start 2.055 3.1218) (end 2.654299 3.721099) (width 0.1524) (layer "F.Cu") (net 16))
 (segment (start 3.5111 5.02635) (end 5.2983 5.02635) (width 0.1524) (layer "F.Cu") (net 15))
 (segment (start 3.1412 4.65645) (end 3.5111 5.02635) (width 0.1524) (layer "F.Cu") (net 15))
 (segment (start 5.2983 5.02635) (end 5.859 4.46565) (width 0.1524) (layer "F.Cu") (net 15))
 (segment (start 2.921706 4) (end 3.1412 4.219494) (width 0.1524) (layer "F.Cu") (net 15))
 (segment (start 1.225 4) (end 2.921706 4) (width 0.1524) (layer "F.Cu") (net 15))
 (segment (start 3.1412 4.219494) (end 3.1412 4.65645) (width 0.1524) (layer "F.Cu") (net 15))
 (segment (start -2.6416 4.497) (end -1.9812 3.8366) (width 0.1524) (layer "F.Cu") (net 2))
 (segment (start -0.5282 3.1218) (end -0.5 3.15) (width 0.1524) (layer "F.Cu") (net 2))
 (segment (start -3.8862 3.5814) (end -3.8862 4.2672) (width 0.1524) (layer "F.Cu") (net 2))
 (segment (start -3.8862 4.2672) (end -3.683 4.4704) (width 0.1524) (layer "F.Cu") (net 2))
 (segment (start -3.9116 3.556) (end -3.8862 3.5814) (width 0.1524) (layer "F.Cu") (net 2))
 (segment (start -1.9812 3.8366) (end -1.9812 3.320088) (width 0.1524) (layer "F.Cu") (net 2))
 (segment (start -1.9812 3.320088) (end -1.782912 3.1218) (width 0.1524) (layer "F.Cu") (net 2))
 (segment (start -3.683 4.4704) (end -2.6682 4.4704) (width 0.1524) (layer "F.Cu") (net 2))
 (segment (start -1.782912 3.1218) (end -0.5282 3.1218) (width 0.1524) (layer "F.Cu") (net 2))
 (segment (start -2.6682 4.4704) (end -2.6416 4.497) (width 0.1524) (layer "F.Cu") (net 2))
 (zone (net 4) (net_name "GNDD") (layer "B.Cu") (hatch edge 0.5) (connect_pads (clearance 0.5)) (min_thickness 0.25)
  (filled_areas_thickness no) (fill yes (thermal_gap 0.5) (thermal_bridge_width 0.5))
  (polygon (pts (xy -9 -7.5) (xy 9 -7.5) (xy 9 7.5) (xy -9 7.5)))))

